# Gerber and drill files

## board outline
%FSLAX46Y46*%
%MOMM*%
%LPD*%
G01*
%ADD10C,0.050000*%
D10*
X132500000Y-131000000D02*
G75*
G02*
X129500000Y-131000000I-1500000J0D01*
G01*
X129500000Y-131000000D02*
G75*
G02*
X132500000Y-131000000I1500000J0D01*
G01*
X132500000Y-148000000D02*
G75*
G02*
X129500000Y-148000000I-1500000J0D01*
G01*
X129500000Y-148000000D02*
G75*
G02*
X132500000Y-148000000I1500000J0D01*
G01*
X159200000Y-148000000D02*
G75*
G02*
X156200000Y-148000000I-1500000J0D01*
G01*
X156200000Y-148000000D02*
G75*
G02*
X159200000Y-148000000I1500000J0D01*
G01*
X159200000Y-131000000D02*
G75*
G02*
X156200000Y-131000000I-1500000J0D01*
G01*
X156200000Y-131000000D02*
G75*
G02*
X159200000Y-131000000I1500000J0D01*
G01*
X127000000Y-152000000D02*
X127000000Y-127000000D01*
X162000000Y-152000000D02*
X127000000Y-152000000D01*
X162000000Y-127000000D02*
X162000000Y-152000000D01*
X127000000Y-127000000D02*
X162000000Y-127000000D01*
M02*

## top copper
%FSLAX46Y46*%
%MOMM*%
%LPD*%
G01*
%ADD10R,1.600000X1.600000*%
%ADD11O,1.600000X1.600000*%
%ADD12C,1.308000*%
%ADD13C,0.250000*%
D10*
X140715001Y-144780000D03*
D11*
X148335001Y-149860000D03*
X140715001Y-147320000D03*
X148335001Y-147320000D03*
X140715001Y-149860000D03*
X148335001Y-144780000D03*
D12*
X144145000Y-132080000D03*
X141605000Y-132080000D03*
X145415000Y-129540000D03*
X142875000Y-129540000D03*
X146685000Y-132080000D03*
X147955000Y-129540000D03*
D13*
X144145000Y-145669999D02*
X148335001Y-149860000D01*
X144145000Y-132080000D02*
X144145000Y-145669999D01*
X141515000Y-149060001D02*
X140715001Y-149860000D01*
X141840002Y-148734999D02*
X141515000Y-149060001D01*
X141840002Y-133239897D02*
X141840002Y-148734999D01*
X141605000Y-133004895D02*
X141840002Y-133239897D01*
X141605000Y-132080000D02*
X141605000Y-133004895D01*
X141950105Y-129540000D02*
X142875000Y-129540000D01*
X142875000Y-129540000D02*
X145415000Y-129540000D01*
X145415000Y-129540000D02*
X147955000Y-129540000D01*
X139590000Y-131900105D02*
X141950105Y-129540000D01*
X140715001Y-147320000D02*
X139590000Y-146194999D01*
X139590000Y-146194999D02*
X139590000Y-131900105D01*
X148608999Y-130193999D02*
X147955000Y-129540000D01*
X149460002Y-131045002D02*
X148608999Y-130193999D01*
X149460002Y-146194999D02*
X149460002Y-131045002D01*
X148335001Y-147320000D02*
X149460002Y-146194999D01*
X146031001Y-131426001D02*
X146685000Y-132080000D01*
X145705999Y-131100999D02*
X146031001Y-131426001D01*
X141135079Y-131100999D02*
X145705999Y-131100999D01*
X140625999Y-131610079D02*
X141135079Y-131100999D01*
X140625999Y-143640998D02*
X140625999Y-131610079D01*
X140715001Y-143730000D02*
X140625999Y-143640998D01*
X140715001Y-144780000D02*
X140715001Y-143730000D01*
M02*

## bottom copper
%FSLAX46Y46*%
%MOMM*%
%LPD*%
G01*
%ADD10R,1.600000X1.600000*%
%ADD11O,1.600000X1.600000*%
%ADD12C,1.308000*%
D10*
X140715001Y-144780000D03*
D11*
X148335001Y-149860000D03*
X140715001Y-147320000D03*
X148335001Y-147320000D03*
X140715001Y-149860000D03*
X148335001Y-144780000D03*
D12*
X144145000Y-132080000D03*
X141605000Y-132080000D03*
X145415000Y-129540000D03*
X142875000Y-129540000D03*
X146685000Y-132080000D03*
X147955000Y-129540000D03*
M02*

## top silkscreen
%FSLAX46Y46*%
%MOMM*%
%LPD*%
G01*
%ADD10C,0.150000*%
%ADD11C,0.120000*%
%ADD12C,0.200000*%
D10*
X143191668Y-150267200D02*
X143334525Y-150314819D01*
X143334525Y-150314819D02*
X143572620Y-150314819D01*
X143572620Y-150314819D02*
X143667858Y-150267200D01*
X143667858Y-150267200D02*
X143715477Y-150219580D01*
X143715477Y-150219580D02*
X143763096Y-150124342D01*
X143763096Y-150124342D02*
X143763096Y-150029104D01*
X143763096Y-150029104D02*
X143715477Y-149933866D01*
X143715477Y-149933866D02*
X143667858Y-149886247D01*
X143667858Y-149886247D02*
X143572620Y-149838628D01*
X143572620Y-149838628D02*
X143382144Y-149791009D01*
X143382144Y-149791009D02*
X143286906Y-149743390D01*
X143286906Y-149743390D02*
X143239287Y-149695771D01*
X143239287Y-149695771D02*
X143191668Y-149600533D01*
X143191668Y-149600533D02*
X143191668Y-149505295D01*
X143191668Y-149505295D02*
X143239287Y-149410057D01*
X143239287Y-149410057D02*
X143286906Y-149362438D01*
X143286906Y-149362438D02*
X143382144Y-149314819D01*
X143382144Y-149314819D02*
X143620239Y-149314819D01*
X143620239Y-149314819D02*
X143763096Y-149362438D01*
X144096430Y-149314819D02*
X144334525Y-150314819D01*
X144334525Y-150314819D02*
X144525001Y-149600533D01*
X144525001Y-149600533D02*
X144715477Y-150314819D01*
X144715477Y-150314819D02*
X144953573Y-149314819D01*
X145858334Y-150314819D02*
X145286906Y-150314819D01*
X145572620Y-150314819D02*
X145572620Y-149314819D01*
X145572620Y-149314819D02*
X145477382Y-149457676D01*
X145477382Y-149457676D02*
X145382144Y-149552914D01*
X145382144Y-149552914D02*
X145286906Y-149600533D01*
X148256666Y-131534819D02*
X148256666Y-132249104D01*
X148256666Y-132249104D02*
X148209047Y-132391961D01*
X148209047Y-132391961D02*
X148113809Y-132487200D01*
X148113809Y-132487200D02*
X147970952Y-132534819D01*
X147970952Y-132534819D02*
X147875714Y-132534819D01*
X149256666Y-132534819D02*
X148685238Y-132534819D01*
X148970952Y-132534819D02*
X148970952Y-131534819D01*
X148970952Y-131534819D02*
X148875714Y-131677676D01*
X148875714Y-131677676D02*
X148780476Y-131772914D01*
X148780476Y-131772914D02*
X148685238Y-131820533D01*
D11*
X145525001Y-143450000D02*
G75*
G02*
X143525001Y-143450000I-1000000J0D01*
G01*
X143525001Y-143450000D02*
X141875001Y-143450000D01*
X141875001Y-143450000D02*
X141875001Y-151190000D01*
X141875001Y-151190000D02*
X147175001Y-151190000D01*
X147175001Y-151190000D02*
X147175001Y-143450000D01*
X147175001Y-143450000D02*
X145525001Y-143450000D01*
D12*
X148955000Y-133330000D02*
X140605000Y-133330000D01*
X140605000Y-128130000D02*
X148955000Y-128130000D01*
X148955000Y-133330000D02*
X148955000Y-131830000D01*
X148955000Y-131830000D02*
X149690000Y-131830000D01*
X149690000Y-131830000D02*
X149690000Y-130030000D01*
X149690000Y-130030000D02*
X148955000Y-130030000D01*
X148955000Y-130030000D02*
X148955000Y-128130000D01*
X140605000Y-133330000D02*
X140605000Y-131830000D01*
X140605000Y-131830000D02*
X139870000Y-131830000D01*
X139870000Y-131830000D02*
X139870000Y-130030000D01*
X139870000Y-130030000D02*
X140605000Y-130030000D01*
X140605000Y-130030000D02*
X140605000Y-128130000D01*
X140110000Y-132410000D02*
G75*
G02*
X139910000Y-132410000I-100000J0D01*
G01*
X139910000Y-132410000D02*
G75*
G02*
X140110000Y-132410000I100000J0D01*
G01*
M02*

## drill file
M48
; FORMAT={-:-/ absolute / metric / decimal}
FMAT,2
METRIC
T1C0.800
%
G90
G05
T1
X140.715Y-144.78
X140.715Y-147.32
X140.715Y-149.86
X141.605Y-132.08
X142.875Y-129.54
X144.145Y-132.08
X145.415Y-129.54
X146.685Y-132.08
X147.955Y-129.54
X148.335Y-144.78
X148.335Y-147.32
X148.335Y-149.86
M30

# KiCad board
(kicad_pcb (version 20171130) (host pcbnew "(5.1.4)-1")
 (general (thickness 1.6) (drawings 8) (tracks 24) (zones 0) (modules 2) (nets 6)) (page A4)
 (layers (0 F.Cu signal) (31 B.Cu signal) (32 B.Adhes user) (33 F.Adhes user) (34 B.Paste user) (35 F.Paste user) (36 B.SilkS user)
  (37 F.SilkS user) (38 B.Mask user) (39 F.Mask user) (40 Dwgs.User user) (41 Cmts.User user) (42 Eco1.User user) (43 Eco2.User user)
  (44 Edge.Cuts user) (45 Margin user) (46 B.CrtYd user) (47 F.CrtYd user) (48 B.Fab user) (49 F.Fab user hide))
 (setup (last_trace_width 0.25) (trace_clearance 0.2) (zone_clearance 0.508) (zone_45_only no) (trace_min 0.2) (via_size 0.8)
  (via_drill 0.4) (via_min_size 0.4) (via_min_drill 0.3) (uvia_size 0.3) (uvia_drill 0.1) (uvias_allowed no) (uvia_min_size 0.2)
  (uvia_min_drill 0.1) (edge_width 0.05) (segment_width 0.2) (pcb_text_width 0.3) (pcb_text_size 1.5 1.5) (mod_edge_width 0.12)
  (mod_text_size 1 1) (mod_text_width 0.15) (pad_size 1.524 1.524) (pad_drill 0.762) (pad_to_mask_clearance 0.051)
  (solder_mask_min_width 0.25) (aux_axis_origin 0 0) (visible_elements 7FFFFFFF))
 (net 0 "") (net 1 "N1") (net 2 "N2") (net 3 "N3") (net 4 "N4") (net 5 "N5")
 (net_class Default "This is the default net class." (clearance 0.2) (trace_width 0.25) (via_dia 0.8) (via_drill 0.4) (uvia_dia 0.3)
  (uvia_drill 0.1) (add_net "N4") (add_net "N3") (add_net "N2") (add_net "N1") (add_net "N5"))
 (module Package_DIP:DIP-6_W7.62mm (layer F.Cu) (at 140.715001 144.78)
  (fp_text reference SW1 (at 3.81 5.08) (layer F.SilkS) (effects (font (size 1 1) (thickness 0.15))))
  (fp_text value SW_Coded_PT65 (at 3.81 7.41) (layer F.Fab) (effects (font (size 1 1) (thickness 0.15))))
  (fp_arc (start 3.81 -1.33) (end 2.81 -1.33) (angle -180) (layer F.SilkS) (width 0.12))
  (fp_line (start 2.81 -1.33) (end 1.16 -1.33) (layer F.SilkS) (width 0.12))
  (fp_line (start 1.16 -1.33) (end 1.16 6.41) (layer F.SilkS) (width 0.12))
  (fp_line (start 1.16 6.41) (end 6.46 6.41) (layer F.SilkS) (width 0.12))
  (fp_line (start 6.46 6.41) (end 6.46 -1.33) (layer F.SilkS) (width 0.12))
  (fp_line (start 6.46 -1.33) (end 4.81 -1.33) (layer F.SilkS) (width 0.12))
  (pad 1 thru_hole rect (at 0 0) (size 1.6 1.6) (drill 0.8) (layers *.Cu *.Mask) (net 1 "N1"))
  (pad 4 thru_hole oval (at 7.62 5.08) (size 1.6 1.6) (drill 0.8) (layers *.Cu *.Mask) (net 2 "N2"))
  (pad 2 thru_hole oval (at 0 2.54) (size 1.6 1.6) (drill 0.8) (layers *.Cu *.Mask) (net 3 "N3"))
  (pad 5 thru_hole oval (at 7.62 2.54) (size 1.6 1.6) (drill 0.8) (layers *.Cu *.Mask) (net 3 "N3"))
  (pad 3 thru_hole oval (at 0 5.08) (size 1.6 1.6) (drill 0.8) (layers *.Cu *.Mask) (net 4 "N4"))
  (pad 6 thru_hole oval (at 7.62 0) (size 1.6 1.6) (drill 0.8) (layers *.Cu *.Mask) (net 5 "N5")))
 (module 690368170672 (layer F.Cu) (at 144.78 130.81 180)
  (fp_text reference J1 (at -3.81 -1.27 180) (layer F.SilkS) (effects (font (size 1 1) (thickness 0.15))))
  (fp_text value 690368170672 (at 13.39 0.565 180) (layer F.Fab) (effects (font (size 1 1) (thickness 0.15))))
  (fp_line (start -4.175 -2.52) (end 4.175 -2.52) (layer F.SilkS) (width 0.2))
  (fp_line (start 4.175 2.68) (end -4.175 2.68) (layer F.SilkS) (width 0.2))
  (fp_line (start -4.175 -2.52) (end -4.175 -1.02) (layer F.SilkS) (width 0.2))
  (fp_line (start -4.175 -1.02) (end -4.91 -1.02) (layer F.SilkS) (width 0.2))
  (fp_line (start -4.91 -1.02) (end -4.91 0.78) (layer F.SilkS) (width 0.2))
  (fp_line (start -4.91 0.78) (end -4.175 0.78) (layer F.SilkS) (width 0.2))
  (fp_line (start -4.175 0.78) (end -4.175 2.68) (layer F.SilkS) (width 0.2))
  (fp_line (start 4.175 -2.52) (end 4.175 -1.02) (layer F.SilkS) (width 0.2))
  (fp_line (start 4.175 -1.02) (end 4.91 -1.02) (layer F.SilkS) (width 0.2))
  (fp_line (start 4.91 -1.02) (end 4.91 0.78) (layer F.SilkS) (width 0.2))
  (fp_line (start 4.91 0.78) (end 4.175 0.78) (layer F.SilkS) (width 0.2))
  (fp_line (start 4.175 0.78) (end 4.175 2.68) (layer F.SilkS) (width 0.2))
  (fp_circle (center 4.77 -1.6) (end 4.87 -1.6) (layer F.SilkS) (width 0.2))
  (pad 3 thru_hole circle (at 0.635 -1.27 180) (size 1.308 1.308) (drill 0.8) (layers *.Cu *.Mask) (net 2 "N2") (solder_mask_margin 0.102))
  (pad 1 thru_hole circle (at 3.175 -1.27 180) (size 1.308 1.308) (drill 0.8) (layers *.Cu *.Mask) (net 4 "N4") (solder_mask_margin 0.102))
  (pad 4 thru_hole circle (at -0.635 1.27 180) (size 1.308 1.308) (drill 0.8) (layers *.Cu *.Mask) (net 3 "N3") (solder_mask_margin 0.102))
  (pad 2 thru_hole circle (at 1.905 1.27 180) (size 1.308 1.308) (drill 0.8) (layers *.Cu *.Mask) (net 3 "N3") (solder_mask_margin 0.102))
  (pad 5 thru_hole circle (at -1.905 -1.27 180) (size 1.308 1.308) (drill 0.8) (layers *.Cu *.Mask) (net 1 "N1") (solder_mask_margin 0.102))
  (pad 6 thru_hole circle (at -3.175 1.27 180) (size 1.308 1.308) (drill 0.8) (layers *.Cu *.Mask) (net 3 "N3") (solder_mask_margin 0.102)))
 (gr_circle (center 131 131) (end 132.5 131) (layer Edge.Cuts) (width 0.05))
 (gr_circle (center 131 148) (end 132.5 148) (layer Edge.Cuts) (width 0.05))
 (gr_circle (center 157.7 148) (end 159.2 148) (layer Edge.Cuts) (width 0.05))
 (gr_circle (center 157.7 131) (end 159.2 131) (layer Edge.Cuts) (width 0.05))
 (gr_line (start 127 152) (end 127 127) (layer Edge.Cuts) (width 0.05))
 (gr_line (start 162 152) (end 127 152) (layer Edge.Cuts) (width 0.05))
 (gr_line (start 162 127) (end 162 152) (layer Edge.Cuts) (width 0.05))
 (gr_line (start 127 127) (end 162 127) (layer Edge.Cuts) (width 0.05))
 (segment (start 144.145 145.669999) (end 148.335001 149.86) (width 0.25) (layer F.Cu) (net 2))
 (segment (start 144.145 132.08) (end 144.145 145.669999) (width 0.25) (layer F.Cu) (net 2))
 (segment (start 141.515 149.060001) (end 140.715001 149.86) (width 0.25) (layer F.Cu) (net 4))
 (segment (start 141.840002 148.734999) (end 141.515 149.060001) (width 0.25) (layer F.Cu) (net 4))
 (segment (start 141.840002 133.239897) (end 141.840002 148.734999) (width 0.25) (layer F.Cu) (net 4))
 (segment (start 141.605 133.004895) (end 141.840002 133.239897) (width 0.25) (layer F.Cu) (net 4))
 (segment (start 141.605 132.08) (end 141.605 133.004895) (width 0.25) (layer F.Cu) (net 4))
 (segment (start 141.950105 129.54) (end 142.875 129.54) (width 0.25) (layer F.Cu) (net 3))
 (segment (start 142.875 129.54) (end 145.415 129.54) (width 0.25) (layer F.Cu) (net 3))
 (segment (start 145.415 129.54) (end 147.955 129.54) (width 0.25) (layer F.Cu) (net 3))
 (segment (start 139.59 131.900105) (end 141.950105 129.54) (width 0.25) (layer F.Cu) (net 3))
 (segment (start 140.715001 147.32) (end 139.59 146.194999) (width 0.25) (layer F.Cu) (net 3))
 (segment (start 139.59 146.194999) (end 139.59 131.900105) (width 0.25) (layer F.Cu) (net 3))
 (segment (start 148.608999 130.193999) (end 147.955 129.54) (width 0.25) (layer F.Cu) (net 3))
 (segment (start 149.460002 131.045002) (end 148.608999 130.193999) (width 0.25) (layer F.Cu) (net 3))
 (segment (start 149.460002 146.194999) (end 149.460002 131.045002) (width 0.25) (layer F.Cu) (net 3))
 (segment (start 148.335001 147.32) (end 149.460002 146.194999) (width 0.25) (layer F.Cu) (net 3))
 (segment (start 146.031001 131.426001) (end 146.685 132.08) (width 0.25) (layer F.Cu) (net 1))
 (segment (start 145.705999 131.100999) (end 146.031001 131.426001) (width 0.25) (layer F.Cu) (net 1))
 (segment (start 141.135079 131.100999) (end 145.705999 131.100999) (width 0.25) (layer F.Cu) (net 1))
 (segment (start 140.625999 131.610079) (end 141.135079 131.100999) (width 0.25) (layer F.Cu) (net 1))
 (segment (start 140.625999 143.640998) (end 140.625999 131.610079) (width 0.25) (layer F.Cu) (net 1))
 (segment (start 140.715001 143.73) (end 140.625999 143.640998) (width 0.25) (layer F.Cu) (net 1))
 (segment (start 140.715001 144.78) (end 140.715001 143.73) (width 0.25) (layer F.Cu) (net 1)))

